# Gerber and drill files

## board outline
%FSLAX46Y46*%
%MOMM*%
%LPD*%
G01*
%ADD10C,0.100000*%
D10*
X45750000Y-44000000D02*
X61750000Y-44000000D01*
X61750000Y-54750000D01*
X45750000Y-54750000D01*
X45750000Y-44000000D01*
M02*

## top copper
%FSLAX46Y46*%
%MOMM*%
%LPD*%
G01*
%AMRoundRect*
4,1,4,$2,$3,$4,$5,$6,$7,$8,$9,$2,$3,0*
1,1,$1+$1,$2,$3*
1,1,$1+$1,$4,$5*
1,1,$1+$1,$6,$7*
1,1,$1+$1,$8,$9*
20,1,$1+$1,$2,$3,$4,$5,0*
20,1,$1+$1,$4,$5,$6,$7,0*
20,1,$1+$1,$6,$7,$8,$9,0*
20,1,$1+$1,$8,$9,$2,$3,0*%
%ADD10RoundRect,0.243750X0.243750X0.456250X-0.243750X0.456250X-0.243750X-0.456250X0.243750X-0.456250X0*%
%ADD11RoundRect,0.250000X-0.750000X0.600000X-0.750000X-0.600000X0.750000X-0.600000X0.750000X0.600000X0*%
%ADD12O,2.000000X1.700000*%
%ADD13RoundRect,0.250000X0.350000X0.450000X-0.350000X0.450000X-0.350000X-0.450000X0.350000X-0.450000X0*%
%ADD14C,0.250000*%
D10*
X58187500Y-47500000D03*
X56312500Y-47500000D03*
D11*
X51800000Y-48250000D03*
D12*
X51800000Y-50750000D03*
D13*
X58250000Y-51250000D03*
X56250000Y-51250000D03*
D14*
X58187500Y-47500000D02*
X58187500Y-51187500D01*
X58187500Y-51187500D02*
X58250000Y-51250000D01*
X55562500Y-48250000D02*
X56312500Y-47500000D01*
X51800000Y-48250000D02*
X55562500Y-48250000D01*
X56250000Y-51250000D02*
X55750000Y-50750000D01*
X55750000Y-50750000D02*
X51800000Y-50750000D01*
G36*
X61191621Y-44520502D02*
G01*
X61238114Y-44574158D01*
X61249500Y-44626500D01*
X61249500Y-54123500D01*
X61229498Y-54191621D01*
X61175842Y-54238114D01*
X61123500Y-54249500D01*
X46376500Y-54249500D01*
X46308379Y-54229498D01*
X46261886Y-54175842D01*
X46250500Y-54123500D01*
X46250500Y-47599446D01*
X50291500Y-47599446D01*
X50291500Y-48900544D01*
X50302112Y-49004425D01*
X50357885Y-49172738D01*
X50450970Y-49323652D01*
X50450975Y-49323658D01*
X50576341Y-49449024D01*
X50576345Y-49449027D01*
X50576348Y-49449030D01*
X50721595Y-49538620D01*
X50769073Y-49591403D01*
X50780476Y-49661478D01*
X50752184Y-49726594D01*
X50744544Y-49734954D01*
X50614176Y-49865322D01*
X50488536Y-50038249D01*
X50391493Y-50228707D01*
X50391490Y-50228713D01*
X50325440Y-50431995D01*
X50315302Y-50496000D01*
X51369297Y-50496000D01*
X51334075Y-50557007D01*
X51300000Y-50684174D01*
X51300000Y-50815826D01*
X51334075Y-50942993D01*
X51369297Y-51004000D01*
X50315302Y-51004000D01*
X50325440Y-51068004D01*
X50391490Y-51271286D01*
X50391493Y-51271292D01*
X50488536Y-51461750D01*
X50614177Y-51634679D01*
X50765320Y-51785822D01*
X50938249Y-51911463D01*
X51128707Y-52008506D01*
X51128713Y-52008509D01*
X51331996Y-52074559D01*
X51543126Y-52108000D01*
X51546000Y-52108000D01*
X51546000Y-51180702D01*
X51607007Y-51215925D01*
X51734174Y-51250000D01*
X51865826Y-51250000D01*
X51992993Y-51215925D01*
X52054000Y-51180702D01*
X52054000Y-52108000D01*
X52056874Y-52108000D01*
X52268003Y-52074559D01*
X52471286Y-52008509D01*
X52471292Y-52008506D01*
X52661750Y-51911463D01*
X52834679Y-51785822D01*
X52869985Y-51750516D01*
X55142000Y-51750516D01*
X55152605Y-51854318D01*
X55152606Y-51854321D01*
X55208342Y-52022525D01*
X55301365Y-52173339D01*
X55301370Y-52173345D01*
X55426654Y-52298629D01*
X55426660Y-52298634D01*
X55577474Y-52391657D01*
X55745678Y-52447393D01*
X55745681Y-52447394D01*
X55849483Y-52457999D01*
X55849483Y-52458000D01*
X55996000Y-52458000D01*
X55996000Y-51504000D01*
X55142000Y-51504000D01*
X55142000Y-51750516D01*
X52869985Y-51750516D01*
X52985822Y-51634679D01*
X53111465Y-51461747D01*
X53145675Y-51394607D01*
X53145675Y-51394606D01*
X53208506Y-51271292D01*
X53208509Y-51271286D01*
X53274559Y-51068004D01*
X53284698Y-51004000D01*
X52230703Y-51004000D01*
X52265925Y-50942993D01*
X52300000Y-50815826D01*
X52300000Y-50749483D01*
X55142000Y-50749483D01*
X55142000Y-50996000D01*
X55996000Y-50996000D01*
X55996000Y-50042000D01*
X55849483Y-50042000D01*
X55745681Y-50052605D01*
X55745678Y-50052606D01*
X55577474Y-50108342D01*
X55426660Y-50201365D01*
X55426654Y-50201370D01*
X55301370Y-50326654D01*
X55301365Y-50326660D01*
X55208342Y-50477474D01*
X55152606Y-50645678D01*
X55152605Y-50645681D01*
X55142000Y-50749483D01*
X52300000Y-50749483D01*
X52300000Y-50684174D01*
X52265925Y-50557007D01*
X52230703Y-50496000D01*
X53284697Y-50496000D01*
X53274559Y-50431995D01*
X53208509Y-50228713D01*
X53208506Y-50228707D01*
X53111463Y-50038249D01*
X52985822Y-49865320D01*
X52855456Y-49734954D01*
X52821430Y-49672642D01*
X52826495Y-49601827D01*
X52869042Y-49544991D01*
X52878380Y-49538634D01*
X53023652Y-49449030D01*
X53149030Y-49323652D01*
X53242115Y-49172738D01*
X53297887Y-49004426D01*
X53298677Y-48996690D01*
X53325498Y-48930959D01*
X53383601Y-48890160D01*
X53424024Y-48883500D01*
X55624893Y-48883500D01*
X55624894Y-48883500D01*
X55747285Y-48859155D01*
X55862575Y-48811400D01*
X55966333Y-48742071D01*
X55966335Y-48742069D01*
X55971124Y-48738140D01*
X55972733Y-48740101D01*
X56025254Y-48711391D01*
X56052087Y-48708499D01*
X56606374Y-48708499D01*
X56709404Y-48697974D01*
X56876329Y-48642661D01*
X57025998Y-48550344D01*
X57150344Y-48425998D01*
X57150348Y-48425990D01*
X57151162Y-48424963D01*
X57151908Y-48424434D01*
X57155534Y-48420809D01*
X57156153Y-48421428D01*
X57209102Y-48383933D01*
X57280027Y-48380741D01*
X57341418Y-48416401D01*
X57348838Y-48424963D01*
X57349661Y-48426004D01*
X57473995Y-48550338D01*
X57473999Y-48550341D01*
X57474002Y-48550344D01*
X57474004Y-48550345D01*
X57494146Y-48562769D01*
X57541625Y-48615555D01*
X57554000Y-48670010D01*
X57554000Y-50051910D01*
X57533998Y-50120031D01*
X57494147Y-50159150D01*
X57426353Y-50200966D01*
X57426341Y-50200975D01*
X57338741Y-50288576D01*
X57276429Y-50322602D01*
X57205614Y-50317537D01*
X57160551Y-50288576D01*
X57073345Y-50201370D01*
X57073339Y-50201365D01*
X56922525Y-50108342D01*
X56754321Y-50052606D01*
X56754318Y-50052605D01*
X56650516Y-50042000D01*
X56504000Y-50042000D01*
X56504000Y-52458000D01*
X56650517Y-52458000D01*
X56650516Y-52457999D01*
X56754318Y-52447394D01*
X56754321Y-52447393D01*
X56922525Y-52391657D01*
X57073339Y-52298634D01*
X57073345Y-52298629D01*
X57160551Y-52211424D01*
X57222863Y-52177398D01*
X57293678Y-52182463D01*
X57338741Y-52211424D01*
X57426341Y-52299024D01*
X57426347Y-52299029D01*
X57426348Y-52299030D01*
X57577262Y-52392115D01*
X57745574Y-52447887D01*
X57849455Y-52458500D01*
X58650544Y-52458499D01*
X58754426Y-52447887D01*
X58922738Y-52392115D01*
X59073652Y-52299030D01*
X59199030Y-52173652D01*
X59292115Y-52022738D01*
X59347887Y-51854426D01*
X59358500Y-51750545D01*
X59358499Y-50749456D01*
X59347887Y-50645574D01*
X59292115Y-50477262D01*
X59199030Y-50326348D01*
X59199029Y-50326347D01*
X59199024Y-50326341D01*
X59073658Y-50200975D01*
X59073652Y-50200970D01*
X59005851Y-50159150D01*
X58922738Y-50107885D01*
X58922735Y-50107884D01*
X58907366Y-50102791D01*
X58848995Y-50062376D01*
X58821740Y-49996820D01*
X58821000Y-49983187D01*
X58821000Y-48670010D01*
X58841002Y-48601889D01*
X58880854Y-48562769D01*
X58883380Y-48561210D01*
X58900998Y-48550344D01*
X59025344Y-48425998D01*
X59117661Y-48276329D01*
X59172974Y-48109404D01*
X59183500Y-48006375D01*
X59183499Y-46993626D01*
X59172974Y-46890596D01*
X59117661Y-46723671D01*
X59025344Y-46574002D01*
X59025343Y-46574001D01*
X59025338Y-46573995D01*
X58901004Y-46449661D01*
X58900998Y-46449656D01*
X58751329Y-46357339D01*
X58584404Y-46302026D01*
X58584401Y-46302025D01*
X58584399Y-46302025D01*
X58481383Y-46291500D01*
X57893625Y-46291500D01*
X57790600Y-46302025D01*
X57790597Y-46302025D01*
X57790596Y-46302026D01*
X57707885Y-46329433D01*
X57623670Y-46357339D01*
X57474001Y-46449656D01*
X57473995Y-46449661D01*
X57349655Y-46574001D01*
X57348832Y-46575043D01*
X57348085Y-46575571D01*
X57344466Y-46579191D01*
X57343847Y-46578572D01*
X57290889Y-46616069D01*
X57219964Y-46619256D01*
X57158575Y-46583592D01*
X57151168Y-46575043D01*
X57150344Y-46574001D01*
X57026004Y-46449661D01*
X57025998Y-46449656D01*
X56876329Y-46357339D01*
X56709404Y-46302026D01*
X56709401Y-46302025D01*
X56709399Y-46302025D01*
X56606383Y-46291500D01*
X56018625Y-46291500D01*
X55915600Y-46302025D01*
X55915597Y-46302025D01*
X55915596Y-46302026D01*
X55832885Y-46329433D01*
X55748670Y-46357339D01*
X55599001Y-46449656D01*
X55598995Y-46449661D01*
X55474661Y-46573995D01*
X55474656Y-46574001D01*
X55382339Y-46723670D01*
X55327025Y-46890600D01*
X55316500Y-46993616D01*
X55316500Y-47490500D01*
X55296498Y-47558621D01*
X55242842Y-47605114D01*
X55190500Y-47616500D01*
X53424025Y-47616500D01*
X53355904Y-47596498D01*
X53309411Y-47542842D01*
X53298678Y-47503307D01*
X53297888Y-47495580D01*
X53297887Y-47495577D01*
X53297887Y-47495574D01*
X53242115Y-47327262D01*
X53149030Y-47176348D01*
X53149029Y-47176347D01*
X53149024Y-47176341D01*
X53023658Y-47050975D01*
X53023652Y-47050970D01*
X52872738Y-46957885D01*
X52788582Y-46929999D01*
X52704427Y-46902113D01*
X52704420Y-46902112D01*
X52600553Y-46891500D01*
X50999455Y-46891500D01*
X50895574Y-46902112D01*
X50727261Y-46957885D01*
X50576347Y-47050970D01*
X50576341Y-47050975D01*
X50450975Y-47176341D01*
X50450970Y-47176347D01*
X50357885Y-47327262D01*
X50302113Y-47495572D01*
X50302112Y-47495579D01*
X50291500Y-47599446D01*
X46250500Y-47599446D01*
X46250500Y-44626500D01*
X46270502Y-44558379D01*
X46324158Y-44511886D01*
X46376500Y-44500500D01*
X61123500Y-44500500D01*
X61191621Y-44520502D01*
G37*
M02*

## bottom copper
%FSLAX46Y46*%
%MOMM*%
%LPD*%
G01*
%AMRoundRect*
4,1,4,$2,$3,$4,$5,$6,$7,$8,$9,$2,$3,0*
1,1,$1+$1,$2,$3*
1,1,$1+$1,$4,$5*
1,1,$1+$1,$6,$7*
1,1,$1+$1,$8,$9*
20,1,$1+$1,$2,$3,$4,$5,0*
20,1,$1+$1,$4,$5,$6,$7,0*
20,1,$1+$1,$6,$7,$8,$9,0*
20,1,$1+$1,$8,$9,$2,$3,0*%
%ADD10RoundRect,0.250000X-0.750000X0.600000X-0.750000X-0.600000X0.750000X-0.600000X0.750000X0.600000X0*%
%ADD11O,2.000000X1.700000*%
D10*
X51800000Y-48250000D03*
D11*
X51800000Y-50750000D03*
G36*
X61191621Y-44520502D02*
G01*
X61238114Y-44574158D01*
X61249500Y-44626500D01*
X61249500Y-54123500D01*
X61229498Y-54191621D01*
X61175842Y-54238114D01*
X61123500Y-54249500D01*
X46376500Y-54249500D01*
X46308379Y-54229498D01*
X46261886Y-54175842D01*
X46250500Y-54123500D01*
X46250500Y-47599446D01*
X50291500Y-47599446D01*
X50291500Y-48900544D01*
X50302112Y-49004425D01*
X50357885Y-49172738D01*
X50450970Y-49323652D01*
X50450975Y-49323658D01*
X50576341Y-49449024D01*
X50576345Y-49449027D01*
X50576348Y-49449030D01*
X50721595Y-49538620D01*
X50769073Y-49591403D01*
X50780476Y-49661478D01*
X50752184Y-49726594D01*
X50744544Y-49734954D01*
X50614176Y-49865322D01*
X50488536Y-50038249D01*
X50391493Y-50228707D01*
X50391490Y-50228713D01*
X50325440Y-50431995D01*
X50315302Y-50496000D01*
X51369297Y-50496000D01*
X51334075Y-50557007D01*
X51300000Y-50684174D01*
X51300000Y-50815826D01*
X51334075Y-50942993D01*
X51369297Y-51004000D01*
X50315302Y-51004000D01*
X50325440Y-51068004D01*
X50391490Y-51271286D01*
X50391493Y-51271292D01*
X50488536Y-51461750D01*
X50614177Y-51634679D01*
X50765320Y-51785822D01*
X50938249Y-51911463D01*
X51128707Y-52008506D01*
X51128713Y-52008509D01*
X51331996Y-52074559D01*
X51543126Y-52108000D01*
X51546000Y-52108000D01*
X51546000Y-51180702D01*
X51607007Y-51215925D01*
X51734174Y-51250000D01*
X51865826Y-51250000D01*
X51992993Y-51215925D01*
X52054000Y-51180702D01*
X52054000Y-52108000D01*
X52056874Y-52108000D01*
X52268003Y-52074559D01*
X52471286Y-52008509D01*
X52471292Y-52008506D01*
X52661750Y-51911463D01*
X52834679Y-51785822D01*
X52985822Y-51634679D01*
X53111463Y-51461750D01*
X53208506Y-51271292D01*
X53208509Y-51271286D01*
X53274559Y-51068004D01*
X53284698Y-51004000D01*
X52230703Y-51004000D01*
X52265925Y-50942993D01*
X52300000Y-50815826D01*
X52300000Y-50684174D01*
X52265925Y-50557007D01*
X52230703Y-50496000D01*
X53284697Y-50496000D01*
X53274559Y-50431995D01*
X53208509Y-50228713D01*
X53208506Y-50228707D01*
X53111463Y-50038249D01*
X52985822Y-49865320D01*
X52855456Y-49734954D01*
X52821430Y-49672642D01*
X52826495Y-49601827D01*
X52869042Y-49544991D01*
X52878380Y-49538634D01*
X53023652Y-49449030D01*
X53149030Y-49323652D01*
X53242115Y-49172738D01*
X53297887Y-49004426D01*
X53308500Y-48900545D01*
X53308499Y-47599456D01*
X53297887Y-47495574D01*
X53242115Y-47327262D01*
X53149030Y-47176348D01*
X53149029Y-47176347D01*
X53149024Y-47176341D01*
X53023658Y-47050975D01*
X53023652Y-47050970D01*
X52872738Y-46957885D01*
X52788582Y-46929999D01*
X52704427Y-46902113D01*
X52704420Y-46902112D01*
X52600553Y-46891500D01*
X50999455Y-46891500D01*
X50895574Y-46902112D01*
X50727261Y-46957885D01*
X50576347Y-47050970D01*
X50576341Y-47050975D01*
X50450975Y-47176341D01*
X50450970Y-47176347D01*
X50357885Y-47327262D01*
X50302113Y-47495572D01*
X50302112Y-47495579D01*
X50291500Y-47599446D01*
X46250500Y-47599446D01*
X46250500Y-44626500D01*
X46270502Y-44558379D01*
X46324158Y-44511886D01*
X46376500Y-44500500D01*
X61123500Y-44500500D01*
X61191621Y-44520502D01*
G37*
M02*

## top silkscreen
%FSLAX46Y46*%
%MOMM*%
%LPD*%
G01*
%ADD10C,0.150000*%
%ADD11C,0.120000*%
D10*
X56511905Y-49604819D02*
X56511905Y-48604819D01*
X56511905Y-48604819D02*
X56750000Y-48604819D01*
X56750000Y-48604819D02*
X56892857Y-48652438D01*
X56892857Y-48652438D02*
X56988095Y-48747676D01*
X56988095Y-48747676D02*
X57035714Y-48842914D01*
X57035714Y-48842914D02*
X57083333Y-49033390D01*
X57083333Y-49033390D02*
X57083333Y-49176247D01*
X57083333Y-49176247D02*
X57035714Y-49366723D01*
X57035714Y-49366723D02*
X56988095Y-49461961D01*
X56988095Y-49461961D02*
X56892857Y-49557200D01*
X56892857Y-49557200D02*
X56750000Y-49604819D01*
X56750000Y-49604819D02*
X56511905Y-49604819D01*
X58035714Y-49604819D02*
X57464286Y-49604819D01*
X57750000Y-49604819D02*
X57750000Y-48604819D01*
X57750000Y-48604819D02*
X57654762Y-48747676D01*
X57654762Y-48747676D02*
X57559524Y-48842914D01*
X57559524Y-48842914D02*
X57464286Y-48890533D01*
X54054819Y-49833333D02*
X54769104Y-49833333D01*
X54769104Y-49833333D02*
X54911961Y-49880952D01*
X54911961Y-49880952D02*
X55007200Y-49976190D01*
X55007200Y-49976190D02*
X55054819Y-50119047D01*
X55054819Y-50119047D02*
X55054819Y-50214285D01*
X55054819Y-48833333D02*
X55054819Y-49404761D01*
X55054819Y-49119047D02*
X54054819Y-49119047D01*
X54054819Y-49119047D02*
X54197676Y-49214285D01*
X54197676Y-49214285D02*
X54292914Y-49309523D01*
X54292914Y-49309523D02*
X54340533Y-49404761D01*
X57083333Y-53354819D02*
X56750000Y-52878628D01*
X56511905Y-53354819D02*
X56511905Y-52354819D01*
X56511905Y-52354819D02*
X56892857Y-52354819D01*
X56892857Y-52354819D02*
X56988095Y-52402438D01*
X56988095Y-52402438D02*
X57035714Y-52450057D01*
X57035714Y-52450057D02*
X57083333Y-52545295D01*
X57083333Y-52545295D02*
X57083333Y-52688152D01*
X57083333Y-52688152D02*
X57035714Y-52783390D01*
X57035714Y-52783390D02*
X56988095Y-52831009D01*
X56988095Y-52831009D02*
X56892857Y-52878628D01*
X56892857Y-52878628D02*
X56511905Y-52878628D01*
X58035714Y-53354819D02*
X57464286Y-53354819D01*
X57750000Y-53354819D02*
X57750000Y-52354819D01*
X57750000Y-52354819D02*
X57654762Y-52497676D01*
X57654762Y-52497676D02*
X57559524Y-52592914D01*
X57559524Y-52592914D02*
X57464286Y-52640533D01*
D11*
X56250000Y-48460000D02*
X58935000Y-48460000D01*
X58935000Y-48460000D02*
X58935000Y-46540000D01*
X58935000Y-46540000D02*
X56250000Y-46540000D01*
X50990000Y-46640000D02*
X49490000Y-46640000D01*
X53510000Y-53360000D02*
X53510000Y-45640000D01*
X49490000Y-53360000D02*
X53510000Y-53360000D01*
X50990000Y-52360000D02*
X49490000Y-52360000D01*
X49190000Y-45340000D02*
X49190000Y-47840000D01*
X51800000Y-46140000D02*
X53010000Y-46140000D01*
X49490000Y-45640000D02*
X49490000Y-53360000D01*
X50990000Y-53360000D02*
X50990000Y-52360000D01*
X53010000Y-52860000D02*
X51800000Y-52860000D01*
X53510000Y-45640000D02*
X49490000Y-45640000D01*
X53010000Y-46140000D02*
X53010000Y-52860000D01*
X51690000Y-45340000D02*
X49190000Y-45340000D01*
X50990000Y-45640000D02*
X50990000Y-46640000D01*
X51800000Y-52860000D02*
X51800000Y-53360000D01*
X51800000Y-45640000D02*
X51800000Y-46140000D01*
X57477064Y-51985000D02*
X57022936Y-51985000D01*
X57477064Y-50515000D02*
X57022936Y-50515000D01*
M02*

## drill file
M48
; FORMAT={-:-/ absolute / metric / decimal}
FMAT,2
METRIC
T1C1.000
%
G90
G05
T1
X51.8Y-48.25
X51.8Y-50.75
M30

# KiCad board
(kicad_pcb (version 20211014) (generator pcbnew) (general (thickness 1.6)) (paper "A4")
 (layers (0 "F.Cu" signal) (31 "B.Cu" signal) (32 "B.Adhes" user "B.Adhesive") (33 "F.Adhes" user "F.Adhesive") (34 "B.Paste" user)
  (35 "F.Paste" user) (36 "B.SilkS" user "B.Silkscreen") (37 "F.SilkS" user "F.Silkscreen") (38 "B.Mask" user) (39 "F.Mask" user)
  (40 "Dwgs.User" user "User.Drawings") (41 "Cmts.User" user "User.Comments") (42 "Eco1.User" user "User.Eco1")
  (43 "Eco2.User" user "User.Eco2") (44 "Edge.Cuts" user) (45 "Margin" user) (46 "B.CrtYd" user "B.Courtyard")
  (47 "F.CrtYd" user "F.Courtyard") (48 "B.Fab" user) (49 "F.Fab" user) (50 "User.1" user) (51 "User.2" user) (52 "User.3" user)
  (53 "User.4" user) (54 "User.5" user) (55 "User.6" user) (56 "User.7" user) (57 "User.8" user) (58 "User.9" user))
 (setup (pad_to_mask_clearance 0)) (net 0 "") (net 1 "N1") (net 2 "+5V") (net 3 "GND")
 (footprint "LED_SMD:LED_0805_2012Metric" (layer "F.Cu") (at 57.25 47.5 180)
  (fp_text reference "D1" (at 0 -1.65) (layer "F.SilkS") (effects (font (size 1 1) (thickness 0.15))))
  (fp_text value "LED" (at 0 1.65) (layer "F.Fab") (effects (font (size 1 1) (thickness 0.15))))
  (fp_line (start 1 -0.96) (end -1.685 -0.96) (layer "F.SilkS") (width 0.12))
  (fp_line (start -1.685 -0.96) (end -1.685 0.96) (layer "F.SilkS") (width 0.12))
  (fp_line (start -1.685 0.96) (end 1 0.96) (layer "F.SilkS") (width 0.12))
  (pad "1" smd roundrect (at -0.9375 0 180) (size 0.975 1.4) (layers "F.Cu" "F.Paste" "F.Mask") (roundrect_rratio 0.25) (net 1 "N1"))
  (pad "2" smd roundrect (at 0.9375 0 180) (size 0.975 1.4) (layers "F.Cu" "F.Paste" "F.Mask") (roundrect_rratio 0.25) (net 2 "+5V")))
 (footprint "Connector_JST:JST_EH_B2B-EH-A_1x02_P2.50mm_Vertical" (layer "F.Cu") (at 51.8 48.25 -90)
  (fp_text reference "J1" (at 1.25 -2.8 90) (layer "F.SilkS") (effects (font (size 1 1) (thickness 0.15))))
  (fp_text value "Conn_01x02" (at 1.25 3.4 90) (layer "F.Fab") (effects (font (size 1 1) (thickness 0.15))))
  (fp_line (start -1.61 0.81) (end -1.61 2.31) (layer "F.SilkS") (width 0.12))
  (fp_line (start 5.11 -1.71) (end -2.61 -1.71) (layer "F.SilkS") (width 0.12))
  (fp_line (start 5.11 2.31) (end 5.11 -1.71) (layer "F.SilkS") (width 0.12))
  (fp_line (start 4.11 0.81) (end 4.11 2.31) (layer "F.SilkS") (width 0.12))
  (fp_line (start -2.91 2.61) (end -0.41 2.61) (layer "F.SilkS") (width 0.12))
  (fp_line (start -2.11 0) (end -2.11 -1.21) (layer "F.SilkS") (width 0.12))
  (fp_line (start -2.61 2.31) (end 5.11 2.31) (layer "F.SilkS") (width 0.12))
  (fp_line (start 5.11 0.81) (end 4.11 0.81) (layer "F.SilkS") (width 0.12))
  (fp_line (start 4.61 -1.21) (end 4.61 0) (layer "F.SilkS") (width 0.12))
  (fp_line (start -2.61 -1.71) (end -2.61 2.31) (layer "F.SilkS") (width 0.12))
  (fp_line (start -2.11 -1.21) (end 4.61 -1.21) (layer "F.SilkS") (width 0.12))
  (fp_line (start -2.91 0.11) (end -2.91 2.61) (layer "F.SilkS") (width 0.12))
  (fp_line (start -2.61 0.81) (end -1.61 0.81) (layer "F.SilkS") (width 0.12))
  (fp_line (start 4.61 0) (end 5.11 0) (layer "F.SilkS") (width 0.12))
  (fp_line (start -2.61 0) (end -2.11 0) (layer "F.SilkS") (width 0.12))
  (pad "1" thru_hole roundrect (at 0 0 270) (size 1.7 2) (drill 1) (layers *.Cu *.Mask) (roundrect_rratio 0.1470588235) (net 2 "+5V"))
  (pad "2" thru_hole oval (at 2.5 0 270) (size 1.7 2) (drill 1) (layers *.Cu *.Mask) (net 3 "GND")))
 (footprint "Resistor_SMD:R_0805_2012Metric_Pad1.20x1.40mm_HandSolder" (layer "F.Cu") (at 57.25 51.25 180)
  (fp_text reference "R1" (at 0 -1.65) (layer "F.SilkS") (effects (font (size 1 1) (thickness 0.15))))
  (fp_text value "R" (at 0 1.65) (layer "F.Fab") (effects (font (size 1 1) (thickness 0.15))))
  (fp_line (start -0.227064 -0.735) (end 0.227064 -0.735) (layer "F.SilkS") (width 0.12))
  (fp_line (start -0.227064 0.735) (end 0.227064 0.735) (layer "F.SilkS") (width 0.12))
  (pad "1" smd roundrect (at -1 0 180) (size 1.2 1.4) (layers "F.Cu" "F.Paste" "F.Mask") (roundrect_rratio 0.2083333333) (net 1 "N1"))
  (pad "2" smd roundrect (at 1 0 180) (size 1.2 1.4) (layers "F.Cu" "F.Paste" "F.Mask") (roundrect_rratio 0.2083333333) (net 3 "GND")))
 (gr_rect (start 61.75 54.75) (end 45.75 44) (layer "Edge.Cuts") (width 0.1) (fill none))
 (segment (start 58.1875 47.5) (end 58.1875 51.1875) (width 0.25) (layer "F.Cu") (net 1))
 (segment (start 58.1875 51.1875) (end 58.25 51.25) (width 0.25) (layer "F.Cu") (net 1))
 (segment (start 55.5625 48.25) (end 56.3125 47.5) (width 0.25) (layer "F.Cu") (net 2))
 (segment (start 51.8 48.25) (end 55.5625 48.25) (width 0.25) (layer "F.Cu") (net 2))
 (segment (start 56.25 51.25) (end 55.75 50.75) (width 0.25) (layer "F.Cu") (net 3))
 (segment (start 55.75 50.75) (end 51.8 50.75) (width 0.25) (layer "F.Cu") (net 3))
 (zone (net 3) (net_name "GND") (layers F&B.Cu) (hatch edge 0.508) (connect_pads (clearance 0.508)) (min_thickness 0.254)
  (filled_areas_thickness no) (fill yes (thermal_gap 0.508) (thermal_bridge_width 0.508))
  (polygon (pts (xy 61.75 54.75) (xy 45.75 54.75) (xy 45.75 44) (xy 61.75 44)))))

